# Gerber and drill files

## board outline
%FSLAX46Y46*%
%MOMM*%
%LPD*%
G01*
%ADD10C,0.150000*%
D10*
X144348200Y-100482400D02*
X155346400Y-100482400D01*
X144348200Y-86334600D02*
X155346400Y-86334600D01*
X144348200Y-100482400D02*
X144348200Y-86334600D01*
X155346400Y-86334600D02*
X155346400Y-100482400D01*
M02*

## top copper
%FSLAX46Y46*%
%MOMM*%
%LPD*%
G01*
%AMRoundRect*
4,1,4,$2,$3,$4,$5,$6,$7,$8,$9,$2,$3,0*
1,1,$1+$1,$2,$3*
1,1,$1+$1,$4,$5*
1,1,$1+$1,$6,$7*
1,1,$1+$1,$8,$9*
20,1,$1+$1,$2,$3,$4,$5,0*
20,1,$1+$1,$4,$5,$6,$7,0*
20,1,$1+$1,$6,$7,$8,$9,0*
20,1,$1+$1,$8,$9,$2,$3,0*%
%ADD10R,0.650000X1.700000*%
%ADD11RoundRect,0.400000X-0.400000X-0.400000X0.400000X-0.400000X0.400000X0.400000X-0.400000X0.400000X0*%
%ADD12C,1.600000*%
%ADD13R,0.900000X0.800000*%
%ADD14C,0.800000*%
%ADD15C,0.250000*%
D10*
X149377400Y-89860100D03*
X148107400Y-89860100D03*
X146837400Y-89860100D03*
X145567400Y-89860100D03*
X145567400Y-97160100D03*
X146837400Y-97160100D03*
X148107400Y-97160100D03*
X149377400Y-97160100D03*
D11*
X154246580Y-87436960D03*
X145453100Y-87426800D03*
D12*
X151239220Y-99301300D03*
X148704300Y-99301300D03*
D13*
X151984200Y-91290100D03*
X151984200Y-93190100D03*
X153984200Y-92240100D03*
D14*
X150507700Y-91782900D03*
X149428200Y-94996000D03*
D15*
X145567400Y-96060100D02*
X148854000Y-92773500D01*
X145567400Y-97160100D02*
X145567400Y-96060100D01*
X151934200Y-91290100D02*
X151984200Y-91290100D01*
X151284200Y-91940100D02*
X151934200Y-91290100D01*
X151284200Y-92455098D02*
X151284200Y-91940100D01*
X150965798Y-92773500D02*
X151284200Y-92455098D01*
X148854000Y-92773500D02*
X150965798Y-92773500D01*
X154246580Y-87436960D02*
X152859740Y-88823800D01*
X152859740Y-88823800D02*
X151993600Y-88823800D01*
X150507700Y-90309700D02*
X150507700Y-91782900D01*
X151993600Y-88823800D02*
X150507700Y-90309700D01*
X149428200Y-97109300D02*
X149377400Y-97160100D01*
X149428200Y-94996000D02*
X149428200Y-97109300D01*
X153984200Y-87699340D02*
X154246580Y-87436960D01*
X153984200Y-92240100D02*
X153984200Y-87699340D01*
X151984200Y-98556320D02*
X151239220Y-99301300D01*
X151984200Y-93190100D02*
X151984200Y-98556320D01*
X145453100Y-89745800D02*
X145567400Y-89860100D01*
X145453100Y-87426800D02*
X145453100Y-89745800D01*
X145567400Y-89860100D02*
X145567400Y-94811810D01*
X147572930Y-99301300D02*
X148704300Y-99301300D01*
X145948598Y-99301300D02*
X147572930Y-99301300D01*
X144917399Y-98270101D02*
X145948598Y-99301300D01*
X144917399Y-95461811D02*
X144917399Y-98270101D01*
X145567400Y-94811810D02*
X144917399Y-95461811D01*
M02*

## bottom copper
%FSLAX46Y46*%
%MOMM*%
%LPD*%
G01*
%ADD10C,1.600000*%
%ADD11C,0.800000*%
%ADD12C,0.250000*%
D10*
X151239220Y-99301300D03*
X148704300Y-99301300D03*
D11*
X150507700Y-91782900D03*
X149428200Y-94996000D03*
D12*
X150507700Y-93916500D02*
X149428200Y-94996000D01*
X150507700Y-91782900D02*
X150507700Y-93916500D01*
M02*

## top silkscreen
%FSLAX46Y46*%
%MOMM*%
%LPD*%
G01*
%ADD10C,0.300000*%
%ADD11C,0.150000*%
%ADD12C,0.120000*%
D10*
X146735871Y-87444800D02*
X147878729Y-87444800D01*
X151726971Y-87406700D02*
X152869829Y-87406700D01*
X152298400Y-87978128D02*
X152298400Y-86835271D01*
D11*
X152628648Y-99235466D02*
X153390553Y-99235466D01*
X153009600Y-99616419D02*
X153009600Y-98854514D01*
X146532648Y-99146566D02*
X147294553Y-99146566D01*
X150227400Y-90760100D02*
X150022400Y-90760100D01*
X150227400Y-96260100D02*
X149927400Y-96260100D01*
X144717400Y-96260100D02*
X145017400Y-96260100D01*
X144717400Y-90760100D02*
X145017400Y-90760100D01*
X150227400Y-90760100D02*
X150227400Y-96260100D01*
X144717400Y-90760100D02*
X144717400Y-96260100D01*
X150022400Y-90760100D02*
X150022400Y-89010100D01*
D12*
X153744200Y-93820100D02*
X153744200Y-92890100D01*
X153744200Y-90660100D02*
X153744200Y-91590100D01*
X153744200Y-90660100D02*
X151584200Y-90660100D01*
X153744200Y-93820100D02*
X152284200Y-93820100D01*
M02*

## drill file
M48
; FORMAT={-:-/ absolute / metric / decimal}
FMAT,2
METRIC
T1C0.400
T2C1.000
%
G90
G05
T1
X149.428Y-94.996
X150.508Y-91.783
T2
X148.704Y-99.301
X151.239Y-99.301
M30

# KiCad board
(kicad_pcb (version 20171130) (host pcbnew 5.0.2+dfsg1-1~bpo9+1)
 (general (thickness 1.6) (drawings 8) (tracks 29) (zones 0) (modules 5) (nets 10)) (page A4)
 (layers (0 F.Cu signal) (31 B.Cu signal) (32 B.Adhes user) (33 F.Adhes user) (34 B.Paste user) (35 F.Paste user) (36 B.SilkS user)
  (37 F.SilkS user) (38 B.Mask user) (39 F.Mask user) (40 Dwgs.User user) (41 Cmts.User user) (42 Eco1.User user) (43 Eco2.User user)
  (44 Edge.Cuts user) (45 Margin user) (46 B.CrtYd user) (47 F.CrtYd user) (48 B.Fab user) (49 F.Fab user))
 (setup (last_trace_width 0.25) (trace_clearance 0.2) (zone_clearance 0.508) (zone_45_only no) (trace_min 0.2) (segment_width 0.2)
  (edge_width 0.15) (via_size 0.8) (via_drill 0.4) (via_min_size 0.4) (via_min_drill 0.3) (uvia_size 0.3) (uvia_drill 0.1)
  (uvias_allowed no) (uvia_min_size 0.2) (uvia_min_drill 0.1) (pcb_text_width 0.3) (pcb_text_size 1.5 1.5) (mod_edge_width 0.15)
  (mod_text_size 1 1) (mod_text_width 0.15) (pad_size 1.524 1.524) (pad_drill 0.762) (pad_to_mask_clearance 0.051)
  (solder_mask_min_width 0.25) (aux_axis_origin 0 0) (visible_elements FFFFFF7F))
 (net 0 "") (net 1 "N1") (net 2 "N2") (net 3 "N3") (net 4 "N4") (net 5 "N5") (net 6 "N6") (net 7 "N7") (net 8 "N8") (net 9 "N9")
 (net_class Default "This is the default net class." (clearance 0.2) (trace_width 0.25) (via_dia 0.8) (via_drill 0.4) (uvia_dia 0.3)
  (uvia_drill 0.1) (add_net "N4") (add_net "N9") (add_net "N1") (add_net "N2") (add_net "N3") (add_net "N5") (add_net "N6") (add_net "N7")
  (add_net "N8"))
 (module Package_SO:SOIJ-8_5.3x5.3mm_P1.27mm (layer F.Cu) (at 147.4724 93.5101 270)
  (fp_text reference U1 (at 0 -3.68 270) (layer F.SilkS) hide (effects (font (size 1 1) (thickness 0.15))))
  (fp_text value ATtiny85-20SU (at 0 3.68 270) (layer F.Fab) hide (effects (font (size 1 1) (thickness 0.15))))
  (fp_line (start -2.75 -2.755) (end -2.75 -2.55) (layer F.SilkS) (width 0.15))
  (fp_line (start 2.75 -2.755) (end 2.75 -2.455) (layer F.SilkS) (width 0.15))
  (fp_line (start 2.75 2.755) (end 2.75 2.455) (layer F.SilkS) (width 0.15))
  (fp_line (start -2.75 2.755) (end -2.75 2.455) (layer F.SilkS) (width 0.15))
  (fp_line (start -2.75 -2.755) (end 2.75 -2.755) (layer F.SilkS) (width 0.15))
  (fp_line (start -2.75 2.755) (end 2.75 2.755) (layer F.SilkS) (width 0.15))
  (fp_line (start -2.75 -2.55) (end -4.5 -2.55) (layer F.SilkS) (width 0.15))
  (pad 1 smd rect (at -3.65 -1.905 270) (size 1.7 0.65) (layers F.Cu F.Paste F.Mask) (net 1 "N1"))
  (pad 2 smd rect (at -3.65 -0.635 270) (size 1.7 0.65) (layers F.Cu F.Paste F.Mask) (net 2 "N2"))
  (pad 3 smd rect (at -3.65 0.635 270) (size 1.7 0.65) (layers F.Cu F.Paste F.Mask) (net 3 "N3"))
  (pad 4 smd rect (at -3.65 1.905 270) (size 1.7 0.65) (layers F.Cu F.Paste F.Mask) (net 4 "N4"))
  (pad 5 smd rect (at 3.65 1.905 270) (size 1.7 0.65) (layers F.Cu F.Paste F.Mask) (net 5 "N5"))
  (pad 6 smd rect (at 3.65 0.635 270) (size 1.7 0.65) (layers F.Cu F.Paste F.Mask) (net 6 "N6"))
  (pad 7 smd rect (at 3.65 -0.635 270) (size 1.7 0.65) (layers F.Cu F.Paste F.Mask) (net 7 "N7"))
  (pad 8 smd rect (at 3.65 -1.905 270) (size 1.7 0.65) (layers F.Cu F.Paste F.Mask) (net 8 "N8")))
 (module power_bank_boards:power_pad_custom (layer F.Cu) (at 154.2669 87.4268)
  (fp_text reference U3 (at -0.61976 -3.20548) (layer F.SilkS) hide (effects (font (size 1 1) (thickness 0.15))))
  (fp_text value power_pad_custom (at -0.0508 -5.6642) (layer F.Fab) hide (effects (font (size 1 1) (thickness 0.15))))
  (pad 1 smd roundrect (at -0.02032 0.01016) (size 1.6 1.6) (layers F.Cu F.Paste F.Mask) (roundrect_rratio 0.25) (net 8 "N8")))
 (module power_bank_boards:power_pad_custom (layer F.Cu) (at 145.47342 87.41664)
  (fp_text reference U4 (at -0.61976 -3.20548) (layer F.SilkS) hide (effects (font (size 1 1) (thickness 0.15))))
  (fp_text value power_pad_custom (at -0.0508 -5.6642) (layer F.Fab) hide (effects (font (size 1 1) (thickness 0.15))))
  (pad 1 smd roundrect (at -0.02032 0.01016) (size 1.6 1.6) (layers F.Cu F.Paste F.Mask) (roundrect_rratio 0.25) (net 4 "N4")))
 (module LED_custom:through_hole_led (layer F.Cu) (at 149.9743 99.3013 180)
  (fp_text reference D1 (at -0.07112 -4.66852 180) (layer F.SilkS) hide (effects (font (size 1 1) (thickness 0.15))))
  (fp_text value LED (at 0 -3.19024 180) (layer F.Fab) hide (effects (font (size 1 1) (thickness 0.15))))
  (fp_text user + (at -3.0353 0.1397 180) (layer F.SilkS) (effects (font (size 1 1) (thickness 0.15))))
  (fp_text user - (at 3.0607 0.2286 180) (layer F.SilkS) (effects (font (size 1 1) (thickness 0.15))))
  (pad 2 thru_hole circle (at -1.26492 0 180) (size 1.6 1.6) (drill 1) (layers *.Cu *.Mask) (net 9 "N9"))
  (pad 1 thru_hole circle (at 1.27 0 180) (size 1.6 1.6) (drill 1) (layers *.Cu *.Mask) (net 4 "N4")))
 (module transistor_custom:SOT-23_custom (layer F.Cu) (at 152.9842 92.2401)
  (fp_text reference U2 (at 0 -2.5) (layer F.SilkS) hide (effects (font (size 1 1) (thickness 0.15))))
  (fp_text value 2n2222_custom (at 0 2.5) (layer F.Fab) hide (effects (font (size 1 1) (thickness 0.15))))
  (fp_line (start 0.76 1.58) (end 0.76 0.65) (layer F.SilkS) (width 0.12))
  (fp_line (start 0.76 -1.58) (end 0.76 -0.65) (layer F.SilkS) (width 0.12))
  (fp_line (start 0.76 -1.58) (end -1.4 -1.58) (layer F.SilkS) (width 0.12))
  (fp_line (start 0.76 1.58) (end -0.7 1.58) (layer F.SilkS) (width 0.12))
  (pad 2 smd rect (at -1 -0.95) (size 0.9 0.8) (layers F.Cu F.Paste F.Mask) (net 5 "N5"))
  (pad 1 smd rect (at -1 0.95) (size 0.9 0.8) (layers F.Cu F.Paste F.Mask) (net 9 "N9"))
  (pad 3 smd rect (at 1 0) (size 0.9 0.8) (layers F.Cu F.Paste F.Mask) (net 8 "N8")))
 (gr_line (start 144.3482 100.4824) (end 155.3464 100.4824) (layer Edge.Cuts) (width 0.15))
 (gr_line (start 144.3482 86.3346) (end 155.3464 86.3346) (layer Edge.Cuts) (width 0.15))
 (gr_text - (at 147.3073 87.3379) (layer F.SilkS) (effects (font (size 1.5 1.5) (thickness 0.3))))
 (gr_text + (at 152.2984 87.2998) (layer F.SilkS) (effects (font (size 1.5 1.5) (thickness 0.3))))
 (gr_line (start 144.3482 100.4824) (end 144.3482 86.3346) (layer Edge.Cuts) (width 0.15))
 (gr_line (start 155.3464 86.3346) (end 155.3464 100.4824) (layer Edge.Cuts) (width 0.15))
 (segment (start 145.5674 96.0601) (end 148.854 92.7735) (width 0.25) (layer F.Cu) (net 5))
 (segment (start 145.5674 97.1601) (end 145.5674 96.0601) (width 0.25) (layer F.Cu) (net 5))
 (segment (start 151.9342 91.2901) (end 151.9842 91.2901) (width 0.25) (layer F.Cu) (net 5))
 (segment (start 151.2842 91.9401) (end 151.9342 91.2901) (width 0.25) (layer F.Cu) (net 5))
 (segment (start 151.2842 92.455098) (end 151.2842 91.9401) (width 0.25) (layer F.Cu) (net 5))
 (segment (start 150.965798 92.7735) (end 151.2842 92.455098) (width 0.25) (layer F.Cu) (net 5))
 (segment (start 148.854 92.7735) (end 150.965798 92.7735) (width 0.25) (layer F.Cu) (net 5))
 (segment (start 154.24658 87.43696) (end 152.85974 88.8238) (width 0.25) (layer F.Cu) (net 8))
 (segment (start 152.85974 88.8238) (end 151.9936 88.8238) (width 0.25) (layer F.Cu) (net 8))
 (segment (start 150.5077 90.3097) (end 150.5077 91.7829) (width 0.25) (layer F.Cu) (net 8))
 (via (at 150.5077 91.7829) (size 0.8) (drill 0.4) (layers F.Cu B.Cu) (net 8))
 (segment (start 151.9936 88.8238) (end 150.5077 90.3097) (width 0.25) (layer F.Cu) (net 8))
 (via (at 149.4282 94.996) (size 0.8) (drill 0.4) (layers F.Cu B.Cu) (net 8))
 (segment (start 150.5077 93.9165) (end 149.4282 94.996) (width 0.25) (layer B.Cu) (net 8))
 (segment (start 150.5077 91.7829) (end 150.5077 93.9165) (width 0.25) (layer B.Cu) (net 8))
 (segment (start 149.4282 97.1093) (end 149.3774 97.1601) (width 0.25) (layer F.Cu) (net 8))
 (segment (start 149.4282 94.996) (end 149.4282 97.1093) (width 0.25) (layer F.Cu) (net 8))
 (segment (start 153.9842 87.69934) (end 154.24658 87.43696) (width 0.25) (layer F.Cu) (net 8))
 (segment (start 153.9842 92.2401) (end 153.9842 87.69934) (width 0.25) (layer F.Cu) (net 8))
 (segment (start 151.9842 98.55632) (end 151.23922 99.3013) (width 0.25) (layer F.Cu) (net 9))
 (segment (start 151.9842 93.1901) (end 151.9842 98.55632) (width 0.25) (layer F.Cu) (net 9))
 (segment (start 145.4531 89.7458) (end 145.5674 89.8601) (width 0.25) (layer F.Cu) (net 4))
 (segment (start 145.4531 87.4268) (end 145.4531 89.7458) (width 0.25) (layer F.Cu) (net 4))
 (segment (start 145.5674 89.8601) (end 145.5674 94.81181) (width 0.25) (layer F.Cu) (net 4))
 (segment (start 147.57293 99.3013) (end 148.7043 99.3013) (width 0.25) (layer F.Cu) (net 4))
 (segment (start 145.948598 99.3013) (end 147.57293 99.3013) (width 0.25) (layer F.Cu) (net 4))
 (segment (start 144.917399 98.270101) (end 145.948598 99.3013) (width 0.25) (layer F.Cu) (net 4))
 (segment (start 144.917399 95.461811) (end 144.917399 98.270101) (width 0.25) (layer F.Cu) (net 4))
 (segment (start 145.5674 94.81181) (end 144.917399 95.461811) (width 0.25) (layer F.Cu) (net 4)))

